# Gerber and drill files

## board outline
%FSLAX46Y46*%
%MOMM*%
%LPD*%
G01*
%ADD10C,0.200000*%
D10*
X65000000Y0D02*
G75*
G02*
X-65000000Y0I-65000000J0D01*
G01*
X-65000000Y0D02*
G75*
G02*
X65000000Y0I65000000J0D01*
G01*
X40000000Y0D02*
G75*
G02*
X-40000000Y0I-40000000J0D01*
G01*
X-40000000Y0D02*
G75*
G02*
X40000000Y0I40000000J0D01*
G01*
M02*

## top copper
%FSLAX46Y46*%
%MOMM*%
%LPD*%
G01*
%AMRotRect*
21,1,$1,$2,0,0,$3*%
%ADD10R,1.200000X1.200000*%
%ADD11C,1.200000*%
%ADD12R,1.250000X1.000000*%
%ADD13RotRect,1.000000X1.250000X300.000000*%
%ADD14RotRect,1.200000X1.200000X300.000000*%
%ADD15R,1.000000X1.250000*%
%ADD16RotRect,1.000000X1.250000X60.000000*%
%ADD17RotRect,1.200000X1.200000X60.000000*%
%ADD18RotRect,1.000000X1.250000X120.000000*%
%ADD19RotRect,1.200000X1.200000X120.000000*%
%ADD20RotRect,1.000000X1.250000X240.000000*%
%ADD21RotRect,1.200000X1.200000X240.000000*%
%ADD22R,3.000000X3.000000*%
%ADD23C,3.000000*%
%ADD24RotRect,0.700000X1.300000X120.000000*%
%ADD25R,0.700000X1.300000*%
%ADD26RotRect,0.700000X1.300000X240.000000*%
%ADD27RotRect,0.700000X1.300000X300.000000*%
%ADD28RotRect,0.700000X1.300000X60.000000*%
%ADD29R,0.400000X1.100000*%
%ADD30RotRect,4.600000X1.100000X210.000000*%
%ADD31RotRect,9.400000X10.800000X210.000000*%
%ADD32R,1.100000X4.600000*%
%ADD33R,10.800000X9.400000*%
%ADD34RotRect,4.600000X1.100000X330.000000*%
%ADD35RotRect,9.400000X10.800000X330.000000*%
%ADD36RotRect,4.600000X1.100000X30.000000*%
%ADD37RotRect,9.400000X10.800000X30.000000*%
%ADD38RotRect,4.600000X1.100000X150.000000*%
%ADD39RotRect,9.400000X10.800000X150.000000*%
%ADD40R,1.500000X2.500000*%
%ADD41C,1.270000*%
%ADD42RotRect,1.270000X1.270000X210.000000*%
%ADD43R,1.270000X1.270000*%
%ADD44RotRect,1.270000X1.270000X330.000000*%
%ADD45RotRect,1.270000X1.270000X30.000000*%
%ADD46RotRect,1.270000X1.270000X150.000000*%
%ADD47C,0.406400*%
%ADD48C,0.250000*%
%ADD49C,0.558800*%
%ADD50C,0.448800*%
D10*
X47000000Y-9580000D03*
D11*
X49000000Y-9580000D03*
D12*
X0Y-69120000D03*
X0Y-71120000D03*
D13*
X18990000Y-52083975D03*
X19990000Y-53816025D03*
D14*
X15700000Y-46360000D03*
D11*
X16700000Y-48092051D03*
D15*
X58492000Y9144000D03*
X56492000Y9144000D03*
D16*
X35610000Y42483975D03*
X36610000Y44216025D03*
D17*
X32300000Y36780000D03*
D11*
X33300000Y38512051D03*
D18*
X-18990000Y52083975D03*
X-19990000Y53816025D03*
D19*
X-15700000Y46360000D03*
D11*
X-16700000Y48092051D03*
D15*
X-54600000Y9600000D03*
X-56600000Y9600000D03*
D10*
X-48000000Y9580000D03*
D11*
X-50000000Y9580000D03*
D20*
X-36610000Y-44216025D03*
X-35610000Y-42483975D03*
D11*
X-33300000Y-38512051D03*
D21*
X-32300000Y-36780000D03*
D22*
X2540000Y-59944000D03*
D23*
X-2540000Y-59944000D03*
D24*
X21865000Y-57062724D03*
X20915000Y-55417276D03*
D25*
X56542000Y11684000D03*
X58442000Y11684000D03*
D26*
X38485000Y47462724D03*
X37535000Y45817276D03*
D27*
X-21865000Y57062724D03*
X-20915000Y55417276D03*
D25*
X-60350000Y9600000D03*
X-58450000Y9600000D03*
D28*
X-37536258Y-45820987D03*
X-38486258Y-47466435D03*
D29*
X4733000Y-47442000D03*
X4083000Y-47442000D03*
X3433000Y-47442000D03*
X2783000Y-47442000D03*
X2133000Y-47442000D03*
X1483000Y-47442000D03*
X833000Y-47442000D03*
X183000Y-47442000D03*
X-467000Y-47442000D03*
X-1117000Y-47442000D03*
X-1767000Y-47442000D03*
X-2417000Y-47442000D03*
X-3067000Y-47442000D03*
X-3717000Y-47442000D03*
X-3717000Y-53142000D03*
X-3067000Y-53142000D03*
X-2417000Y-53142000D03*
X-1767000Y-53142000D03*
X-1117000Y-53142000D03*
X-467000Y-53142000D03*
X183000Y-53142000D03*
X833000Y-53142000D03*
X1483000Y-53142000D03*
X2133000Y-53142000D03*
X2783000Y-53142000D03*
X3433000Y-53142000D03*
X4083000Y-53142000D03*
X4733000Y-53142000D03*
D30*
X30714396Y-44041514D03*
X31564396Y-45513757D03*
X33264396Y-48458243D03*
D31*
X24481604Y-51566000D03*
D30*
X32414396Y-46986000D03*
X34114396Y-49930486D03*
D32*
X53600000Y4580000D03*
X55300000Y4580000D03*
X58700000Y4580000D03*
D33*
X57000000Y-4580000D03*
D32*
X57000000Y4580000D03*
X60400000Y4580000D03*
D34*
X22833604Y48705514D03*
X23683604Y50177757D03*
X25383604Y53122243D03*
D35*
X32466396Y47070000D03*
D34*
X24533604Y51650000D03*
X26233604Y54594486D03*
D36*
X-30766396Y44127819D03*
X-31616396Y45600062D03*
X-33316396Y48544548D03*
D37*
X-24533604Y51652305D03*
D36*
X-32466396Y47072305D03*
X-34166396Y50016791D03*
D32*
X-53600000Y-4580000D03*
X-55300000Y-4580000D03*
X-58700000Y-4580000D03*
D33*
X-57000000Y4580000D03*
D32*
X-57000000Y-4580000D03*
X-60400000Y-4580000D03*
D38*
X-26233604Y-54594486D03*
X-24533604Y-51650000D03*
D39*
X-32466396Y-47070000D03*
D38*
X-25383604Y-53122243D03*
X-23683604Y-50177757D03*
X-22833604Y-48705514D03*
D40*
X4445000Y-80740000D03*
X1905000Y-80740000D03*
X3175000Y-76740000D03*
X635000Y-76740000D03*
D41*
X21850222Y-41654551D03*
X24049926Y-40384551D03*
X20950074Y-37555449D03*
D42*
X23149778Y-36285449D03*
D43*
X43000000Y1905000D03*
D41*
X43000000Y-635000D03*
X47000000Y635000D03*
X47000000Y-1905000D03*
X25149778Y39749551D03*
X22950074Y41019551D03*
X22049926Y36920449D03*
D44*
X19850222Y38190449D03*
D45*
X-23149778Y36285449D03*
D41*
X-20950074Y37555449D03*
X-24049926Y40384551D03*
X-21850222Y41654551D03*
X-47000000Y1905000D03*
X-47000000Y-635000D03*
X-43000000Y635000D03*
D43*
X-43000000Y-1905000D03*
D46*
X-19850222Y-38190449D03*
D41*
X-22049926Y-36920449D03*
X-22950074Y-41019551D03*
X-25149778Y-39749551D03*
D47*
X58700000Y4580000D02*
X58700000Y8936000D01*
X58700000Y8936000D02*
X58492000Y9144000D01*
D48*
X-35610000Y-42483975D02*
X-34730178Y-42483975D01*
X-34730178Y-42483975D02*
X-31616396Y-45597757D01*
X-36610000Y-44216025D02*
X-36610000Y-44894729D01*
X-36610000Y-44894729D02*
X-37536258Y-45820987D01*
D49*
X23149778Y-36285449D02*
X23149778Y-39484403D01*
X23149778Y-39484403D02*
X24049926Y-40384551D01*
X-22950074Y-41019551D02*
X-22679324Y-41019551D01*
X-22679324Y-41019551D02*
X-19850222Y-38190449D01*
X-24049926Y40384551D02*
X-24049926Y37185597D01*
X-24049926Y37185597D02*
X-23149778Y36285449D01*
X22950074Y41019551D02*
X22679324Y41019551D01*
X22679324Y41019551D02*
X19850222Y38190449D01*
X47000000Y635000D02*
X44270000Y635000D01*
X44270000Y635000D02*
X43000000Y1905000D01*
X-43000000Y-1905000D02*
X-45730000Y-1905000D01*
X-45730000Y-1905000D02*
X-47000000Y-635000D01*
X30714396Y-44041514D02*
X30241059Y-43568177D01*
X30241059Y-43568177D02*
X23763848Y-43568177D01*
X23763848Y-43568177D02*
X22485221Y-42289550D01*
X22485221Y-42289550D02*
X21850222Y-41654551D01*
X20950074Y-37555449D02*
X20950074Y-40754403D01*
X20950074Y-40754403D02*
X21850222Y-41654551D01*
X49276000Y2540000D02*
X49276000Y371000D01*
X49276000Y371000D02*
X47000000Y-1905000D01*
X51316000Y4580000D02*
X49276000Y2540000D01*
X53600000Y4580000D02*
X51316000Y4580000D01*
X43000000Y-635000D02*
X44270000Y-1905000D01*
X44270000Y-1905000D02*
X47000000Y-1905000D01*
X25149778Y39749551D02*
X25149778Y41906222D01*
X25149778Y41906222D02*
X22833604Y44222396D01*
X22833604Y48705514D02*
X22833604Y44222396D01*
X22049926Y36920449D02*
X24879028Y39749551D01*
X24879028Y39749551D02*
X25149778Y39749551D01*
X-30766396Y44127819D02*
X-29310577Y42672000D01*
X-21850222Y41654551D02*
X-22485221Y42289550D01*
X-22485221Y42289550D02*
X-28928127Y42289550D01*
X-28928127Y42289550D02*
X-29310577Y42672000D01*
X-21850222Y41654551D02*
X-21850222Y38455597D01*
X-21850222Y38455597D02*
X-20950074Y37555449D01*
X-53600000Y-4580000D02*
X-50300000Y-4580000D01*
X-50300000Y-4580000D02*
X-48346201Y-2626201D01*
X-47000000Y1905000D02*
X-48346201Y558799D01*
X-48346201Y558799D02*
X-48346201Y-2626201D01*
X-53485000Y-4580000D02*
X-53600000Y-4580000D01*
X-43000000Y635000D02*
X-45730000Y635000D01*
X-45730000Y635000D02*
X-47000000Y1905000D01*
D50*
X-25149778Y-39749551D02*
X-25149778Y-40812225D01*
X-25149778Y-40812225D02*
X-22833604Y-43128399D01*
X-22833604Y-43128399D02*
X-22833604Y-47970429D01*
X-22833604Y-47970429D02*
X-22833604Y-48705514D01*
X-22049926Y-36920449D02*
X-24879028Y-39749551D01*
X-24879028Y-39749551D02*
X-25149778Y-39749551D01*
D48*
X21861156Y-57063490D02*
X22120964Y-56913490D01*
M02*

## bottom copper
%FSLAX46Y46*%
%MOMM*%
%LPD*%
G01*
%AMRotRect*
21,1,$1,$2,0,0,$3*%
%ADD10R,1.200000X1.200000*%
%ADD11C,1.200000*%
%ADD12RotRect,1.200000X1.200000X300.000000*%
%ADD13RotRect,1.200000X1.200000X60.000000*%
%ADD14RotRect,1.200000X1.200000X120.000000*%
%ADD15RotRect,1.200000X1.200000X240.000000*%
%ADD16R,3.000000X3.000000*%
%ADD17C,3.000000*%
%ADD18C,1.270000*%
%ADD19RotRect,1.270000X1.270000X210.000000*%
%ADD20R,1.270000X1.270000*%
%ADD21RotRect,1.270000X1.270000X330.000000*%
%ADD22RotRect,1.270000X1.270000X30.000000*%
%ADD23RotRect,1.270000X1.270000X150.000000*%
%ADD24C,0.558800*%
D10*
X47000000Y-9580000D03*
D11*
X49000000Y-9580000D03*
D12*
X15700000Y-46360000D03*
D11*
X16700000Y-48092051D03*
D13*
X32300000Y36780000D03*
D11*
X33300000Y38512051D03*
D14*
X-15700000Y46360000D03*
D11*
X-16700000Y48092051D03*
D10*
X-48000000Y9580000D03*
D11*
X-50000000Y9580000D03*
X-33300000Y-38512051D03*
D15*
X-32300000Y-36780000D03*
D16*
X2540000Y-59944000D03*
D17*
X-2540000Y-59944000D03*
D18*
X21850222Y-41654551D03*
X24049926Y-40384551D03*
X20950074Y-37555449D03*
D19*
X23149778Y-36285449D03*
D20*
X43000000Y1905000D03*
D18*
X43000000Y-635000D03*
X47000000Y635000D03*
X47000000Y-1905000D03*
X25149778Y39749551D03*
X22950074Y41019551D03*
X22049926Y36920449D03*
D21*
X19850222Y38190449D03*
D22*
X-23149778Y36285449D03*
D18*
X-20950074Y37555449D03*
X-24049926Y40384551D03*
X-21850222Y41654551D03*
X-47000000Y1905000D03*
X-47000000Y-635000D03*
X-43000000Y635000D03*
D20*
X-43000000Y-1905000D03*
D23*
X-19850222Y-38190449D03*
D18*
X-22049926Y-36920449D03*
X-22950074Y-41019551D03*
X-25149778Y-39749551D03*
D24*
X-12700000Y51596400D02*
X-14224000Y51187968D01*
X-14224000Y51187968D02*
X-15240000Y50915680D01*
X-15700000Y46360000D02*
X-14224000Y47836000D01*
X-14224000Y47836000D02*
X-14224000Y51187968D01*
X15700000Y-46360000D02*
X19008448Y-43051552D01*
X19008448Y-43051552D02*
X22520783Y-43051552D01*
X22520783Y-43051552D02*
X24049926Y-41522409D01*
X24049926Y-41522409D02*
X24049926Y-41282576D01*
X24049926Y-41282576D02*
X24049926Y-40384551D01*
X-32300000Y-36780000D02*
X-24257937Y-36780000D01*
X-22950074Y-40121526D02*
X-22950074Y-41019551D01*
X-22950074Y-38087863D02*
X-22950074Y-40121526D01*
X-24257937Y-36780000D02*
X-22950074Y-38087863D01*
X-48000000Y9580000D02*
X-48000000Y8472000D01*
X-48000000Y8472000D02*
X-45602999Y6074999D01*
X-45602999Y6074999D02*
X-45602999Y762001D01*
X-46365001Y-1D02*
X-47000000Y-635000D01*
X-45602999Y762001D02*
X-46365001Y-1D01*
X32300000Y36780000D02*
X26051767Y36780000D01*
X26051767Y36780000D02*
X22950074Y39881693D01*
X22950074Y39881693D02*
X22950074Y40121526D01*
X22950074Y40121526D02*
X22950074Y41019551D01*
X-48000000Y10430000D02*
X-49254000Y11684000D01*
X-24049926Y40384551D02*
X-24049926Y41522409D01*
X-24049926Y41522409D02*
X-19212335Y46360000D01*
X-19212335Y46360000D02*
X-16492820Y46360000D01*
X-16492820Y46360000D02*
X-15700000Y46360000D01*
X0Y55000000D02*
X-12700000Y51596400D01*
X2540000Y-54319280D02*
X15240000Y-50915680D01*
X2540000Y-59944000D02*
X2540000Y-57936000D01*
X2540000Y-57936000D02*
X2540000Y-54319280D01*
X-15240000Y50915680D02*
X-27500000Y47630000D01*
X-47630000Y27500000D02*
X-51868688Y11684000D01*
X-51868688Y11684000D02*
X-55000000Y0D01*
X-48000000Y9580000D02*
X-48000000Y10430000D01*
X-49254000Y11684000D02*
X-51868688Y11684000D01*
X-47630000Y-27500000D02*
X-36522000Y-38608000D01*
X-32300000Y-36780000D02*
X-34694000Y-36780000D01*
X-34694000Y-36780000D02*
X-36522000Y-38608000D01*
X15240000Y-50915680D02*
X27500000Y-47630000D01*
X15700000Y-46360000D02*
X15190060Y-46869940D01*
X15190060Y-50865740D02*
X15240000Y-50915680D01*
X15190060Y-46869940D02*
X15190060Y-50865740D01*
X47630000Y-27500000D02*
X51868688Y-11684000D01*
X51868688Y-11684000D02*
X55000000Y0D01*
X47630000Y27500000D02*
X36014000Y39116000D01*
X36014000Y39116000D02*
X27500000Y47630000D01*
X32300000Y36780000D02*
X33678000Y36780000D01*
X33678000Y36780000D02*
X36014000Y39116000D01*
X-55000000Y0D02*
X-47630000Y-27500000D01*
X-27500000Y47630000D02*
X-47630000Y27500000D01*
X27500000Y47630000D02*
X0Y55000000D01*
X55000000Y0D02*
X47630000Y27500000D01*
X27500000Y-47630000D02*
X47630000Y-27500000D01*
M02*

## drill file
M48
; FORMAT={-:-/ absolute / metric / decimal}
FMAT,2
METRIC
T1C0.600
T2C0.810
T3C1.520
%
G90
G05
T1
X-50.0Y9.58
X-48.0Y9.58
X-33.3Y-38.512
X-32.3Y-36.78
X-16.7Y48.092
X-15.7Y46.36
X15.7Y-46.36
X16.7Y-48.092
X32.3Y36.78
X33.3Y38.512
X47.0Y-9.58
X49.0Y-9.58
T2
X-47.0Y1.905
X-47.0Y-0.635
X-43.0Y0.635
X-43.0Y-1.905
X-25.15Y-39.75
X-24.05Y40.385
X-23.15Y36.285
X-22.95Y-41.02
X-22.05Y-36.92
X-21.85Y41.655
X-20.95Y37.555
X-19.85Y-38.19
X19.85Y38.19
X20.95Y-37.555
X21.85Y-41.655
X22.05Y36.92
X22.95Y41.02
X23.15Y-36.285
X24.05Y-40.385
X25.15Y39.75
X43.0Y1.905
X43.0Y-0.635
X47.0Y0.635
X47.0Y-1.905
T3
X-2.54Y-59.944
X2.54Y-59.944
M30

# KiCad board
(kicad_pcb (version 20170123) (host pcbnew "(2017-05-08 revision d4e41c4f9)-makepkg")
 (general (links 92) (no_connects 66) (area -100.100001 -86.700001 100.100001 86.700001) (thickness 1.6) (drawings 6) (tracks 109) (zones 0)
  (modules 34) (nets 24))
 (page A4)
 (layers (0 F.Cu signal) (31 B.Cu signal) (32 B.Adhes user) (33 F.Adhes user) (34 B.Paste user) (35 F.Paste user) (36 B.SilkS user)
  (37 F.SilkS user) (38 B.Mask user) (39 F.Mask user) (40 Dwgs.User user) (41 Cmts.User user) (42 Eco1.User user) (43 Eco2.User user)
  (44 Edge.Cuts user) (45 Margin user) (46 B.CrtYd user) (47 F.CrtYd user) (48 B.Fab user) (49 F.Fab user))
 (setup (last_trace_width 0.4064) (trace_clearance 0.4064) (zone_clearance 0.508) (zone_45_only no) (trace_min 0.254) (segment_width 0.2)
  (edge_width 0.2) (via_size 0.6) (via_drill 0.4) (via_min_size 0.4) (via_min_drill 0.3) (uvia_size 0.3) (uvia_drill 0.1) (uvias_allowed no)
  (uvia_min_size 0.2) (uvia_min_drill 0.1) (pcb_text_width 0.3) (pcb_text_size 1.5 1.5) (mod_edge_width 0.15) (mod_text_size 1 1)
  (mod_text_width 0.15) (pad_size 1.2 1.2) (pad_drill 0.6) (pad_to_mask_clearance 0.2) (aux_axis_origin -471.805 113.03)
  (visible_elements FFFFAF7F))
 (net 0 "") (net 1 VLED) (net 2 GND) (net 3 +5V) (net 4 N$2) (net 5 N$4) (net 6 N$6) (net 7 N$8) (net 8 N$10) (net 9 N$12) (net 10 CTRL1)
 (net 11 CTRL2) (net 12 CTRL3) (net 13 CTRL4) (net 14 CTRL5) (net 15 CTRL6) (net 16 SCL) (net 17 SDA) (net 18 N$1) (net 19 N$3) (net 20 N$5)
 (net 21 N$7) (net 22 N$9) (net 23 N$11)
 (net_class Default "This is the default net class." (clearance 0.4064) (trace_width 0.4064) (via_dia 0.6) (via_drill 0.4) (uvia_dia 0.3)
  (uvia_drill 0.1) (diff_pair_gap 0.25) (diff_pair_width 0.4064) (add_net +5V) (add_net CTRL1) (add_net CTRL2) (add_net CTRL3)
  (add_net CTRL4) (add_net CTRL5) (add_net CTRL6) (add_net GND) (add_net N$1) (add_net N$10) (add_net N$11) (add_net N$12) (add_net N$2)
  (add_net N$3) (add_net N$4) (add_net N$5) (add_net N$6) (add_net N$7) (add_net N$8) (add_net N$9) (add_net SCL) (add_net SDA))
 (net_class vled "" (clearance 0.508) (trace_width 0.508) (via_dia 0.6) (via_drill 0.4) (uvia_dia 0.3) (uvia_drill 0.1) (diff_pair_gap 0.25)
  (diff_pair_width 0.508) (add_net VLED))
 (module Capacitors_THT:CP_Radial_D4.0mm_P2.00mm (layer F.Cu) (at 47 9.58)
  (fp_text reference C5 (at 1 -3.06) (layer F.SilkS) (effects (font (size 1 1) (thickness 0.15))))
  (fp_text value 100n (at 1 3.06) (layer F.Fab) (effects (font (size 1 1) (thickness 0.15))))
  (pad 1 thru_hole rect (at 0 0) (size 1.2 1.2) (drill 0.6) (layers *.Cu *.Mask) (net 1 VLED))
  (pad 2 thru_hole circle (at 2 0) (size 1.2 1.2) (drill 0.6) (layers *.Cu *.Mask) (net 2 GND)))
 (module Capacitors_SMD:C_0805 (layer F.Cu) (at 0 70.12 270)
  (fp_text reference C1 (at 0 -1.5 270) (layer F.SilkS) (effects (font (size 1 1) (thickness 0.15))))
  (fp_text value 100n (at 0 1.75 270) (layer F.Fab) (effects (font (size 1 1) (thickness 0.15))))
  (pad 1 smd rect (at -1 0 270) (size 1 1.25) (layers F.Cu F.Paste F.Mask) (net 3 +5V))
  (pad 2 smd rect (at 1 0 270) (size 1 1.25) (layers F.Cu F.Paste F.Mask) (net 2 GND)))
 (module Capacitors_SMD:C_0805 (layer F.Cu) (at 19.49 52.95 300)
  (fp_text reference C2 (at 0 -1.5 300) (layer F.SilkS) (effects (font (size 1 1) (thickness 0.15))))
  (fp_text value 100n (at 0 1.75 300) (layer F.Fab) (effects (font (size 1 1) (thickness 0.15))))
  (pad 1 smd rect (at -1 0 300) (size 1 1.25) (layers F.Cu F.Paste F.Mask) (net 3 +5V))
  (pad 2 smd rect (at 1 0 300) (size 1 1.25) (layers F.Cu F.Paste F.Mask) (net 2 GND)))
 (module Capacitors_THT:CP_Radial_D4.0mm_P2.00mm (layer F.Cu) (at 15.7 46.36 300)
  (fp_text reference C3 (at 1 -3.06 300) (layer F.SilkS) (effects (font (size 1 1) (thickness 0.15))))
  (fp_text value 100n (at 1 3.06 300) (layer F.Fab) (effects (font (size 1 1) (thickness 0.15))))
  (pad 1 thru_hole rect (at 0 0 300) (size 1.2 1.2) (drill 0.6) (layers *.Cu *.Mask) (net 1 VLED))
  (pad 2 thru_hole circle (at 2 0 300) (size 1.2 1.2) (drill 0.6) (layers *.Cu *.Mask) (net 2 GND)))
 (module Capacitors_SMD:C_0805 (layer F.Cu) (at 57.492 -9.144 180)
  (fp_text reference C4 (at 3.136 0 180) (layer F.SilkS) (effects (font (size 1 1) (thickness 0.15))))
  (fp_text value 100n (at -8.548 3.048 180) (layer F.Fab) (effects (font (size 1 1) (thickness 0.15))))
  (pad 1 smd rect (at -1 0 180) (size 1 1.25) (layers F.Cu F.Paste F.Mask) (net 3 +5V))
  (pad 2 smd rect (at 1 0 180) (size 1 1.25) (layers F.Cu F.Paste F.Mask) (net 2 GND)))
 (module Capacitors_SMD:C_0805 (layer F.Cu) (at 36.11 -43.35 60)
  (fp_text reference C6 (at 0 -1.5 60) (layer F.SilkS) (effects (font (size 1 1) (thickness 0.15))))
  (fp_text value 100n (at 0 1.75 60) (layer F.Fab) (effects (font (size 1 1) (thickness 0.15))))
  (pad 1 smd rect (at -1 0 60) (size 1 1.25) (layers F.Cu F.Paste F.Mask) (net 3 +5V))
  (pad 2 smd rect (at 1 0 60) (size 1 1.25) (layers F.Cu F.Paste F.Mask) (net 2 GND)))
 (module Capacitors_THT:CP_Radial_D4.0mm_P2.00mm (layer F.Cu) (at 32.3 -36.78 60)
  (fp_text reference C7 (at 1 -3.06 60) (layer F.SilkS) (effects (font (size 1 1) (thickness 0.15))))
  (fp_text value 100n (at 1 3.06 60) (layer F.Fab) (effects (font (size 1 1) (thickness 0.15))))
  (pad 1 thru_hole rect (at 0 0 60) (size 1.2 1.2) (drill 0.6) (layers *.Cu *.Mask) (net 1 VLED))
  (pad 2 thru_hole circle (at 2 0 60) (size 1.2 1.2) (drill 0.6) (layers *.Cu *.Mask) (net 2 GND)))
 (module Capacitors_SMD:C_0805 (layer F.Cu) (at -19.49 -52.95 120)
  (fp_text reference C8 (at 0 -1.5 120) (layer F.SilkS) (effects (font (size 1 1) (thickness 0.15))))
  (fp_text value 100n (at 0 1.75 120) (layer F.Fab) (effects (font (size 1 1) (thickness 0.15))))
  (pad 1 smd rect (at -1 0 120) (size 1 1.25) (layers F.Cu F.Paste F.Mask) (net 3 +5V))
  (pad 2 smd rect (at 1 0 120) (size 1 1.25) (layers F.Cu F.Paste F.Mask) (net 2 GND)))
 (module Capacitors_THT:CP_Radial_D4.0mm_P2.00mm (layer F.Cu) (at -15.7 -46.36 120)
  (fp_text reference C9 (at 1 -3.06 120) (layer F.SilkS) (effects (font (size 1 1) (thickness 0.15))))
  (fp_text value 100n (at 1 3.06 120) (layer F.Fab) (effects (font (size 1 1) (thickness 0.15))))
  (pad 1 thru_hole rect (at 0 0 120) (size 1.2 1.2) (drill 0.6) (layers *.Cu *.Mask) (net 1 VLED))
  (pad 2 thru_hole circle (at 2 0 120) (size 1.2 1.2) (drill 0.6) (layers *.Cu *.Mask) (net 2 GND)))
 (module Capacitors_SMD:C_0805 (layer F.Cu) (at -55.6 -9.6 180)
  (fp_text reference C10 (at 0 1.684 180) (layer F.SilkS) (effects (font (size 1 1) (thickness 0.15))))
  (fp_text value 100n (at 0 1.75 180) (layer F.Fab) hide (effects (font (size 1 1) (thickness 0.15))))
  (pad 1 smd rect (at -1 0 180) (size 1 1.25) (layers F.Cu F.Paste F.Mask) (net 3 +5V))
  (pad 2 smd rect (at 1 0 180) (size 1 1.25) (layers F.Cu F.Paste F.Mask) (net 2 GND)))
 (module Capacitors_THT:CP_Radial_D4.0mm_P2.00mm (layer F.Cu) (at -48 -9.58 180)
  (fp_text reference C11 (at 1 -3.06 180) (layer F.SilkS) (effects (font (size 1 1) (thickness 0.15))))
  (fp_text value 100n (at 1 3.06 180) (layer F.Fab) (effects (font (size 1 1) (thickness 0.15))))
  (pad 1 thru_hole rect (at 0 0 180) (size 1.2 1.2) (drill 0.6) (layers *.Cu *.Mask) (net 1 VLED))
  (pad 2 thru_hole circle (at 2 0 180) (size 1.2 1.2) (drill 0.6) (layers *.Cu *.Mask) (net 2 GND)))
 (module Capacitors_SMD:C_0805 (layer F.Cu) (at -36.11 43.35 240)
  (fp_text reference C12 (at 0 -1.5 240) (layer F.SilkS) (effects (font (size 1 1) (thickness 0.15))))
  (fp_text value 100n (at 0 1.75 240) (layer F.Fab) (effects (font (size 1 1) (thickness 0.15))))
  (pad 2 smd rect (at 1 0 240) (size 1 1.25) (layers F.Cu F.Paste F.Mask) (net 2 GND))
  (pad 1 smd rect (at -1 0 240) (size 1 1.25) (layers F.Cu F.Paste F.Mask) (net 3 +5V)))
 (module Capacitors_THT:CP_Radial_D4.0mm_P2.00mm (layer F.Cu) (at -32.3 36.78 240)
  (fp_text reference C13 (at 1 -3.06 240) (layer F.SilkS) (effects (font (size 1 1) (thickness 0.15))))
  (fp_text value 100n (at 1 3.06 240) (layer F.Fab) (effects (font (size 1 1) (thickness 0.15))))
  (pad 2 thru_hole circle (at 2 0 240) (size 1.2 1.2) (drill 0.6) (layers *.Cu *.Mask) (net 2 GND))
  (pad 1 thru_hole rect (at 0 0 240) (size 1.2 1.2) (drill 0.6) (layers *.Cu *.Mask) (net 1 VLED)))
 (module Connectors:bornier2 (layer F.Cu) (at 2.54 59.944 180)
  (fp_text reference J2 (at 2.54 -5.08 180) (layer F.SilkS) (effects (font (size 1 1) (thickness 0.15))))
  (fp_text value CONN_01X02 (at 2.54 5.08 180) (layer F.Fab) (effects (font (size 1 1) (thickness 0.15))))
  (pad 1 thru_hole rect (at 0 0 180) (size 3 3) (drill 1.52) (layers *.Cu *.Mask) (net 1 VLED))
  (pad 2 thru_hole circle (at 5.08 0 180) (size 3 3) (drill 1.52) (layers *.Cu *.Mask) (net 2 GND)))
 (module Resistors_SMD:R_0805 (layer F.Cu) (at 21.39 56.24 120)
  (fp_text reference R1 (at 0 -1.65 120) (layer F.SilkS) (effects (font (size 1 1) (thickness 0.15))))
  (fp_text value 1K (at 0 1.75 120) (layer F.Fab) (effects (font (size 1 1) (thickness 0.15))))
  (pad 1 smd rect (at -0.95 0 120) (size 0.7 1.3) (layers F.Cu F.Paste F.Mask) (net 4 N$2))
  (pad 2 smd rect (at 0.95 0 120) (size 0.7 1.3) (layers F.Cu F.Paste F.Mask) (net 2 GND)))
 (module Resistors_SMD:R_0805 (layer F.Cu) (at 57.492 -11.684)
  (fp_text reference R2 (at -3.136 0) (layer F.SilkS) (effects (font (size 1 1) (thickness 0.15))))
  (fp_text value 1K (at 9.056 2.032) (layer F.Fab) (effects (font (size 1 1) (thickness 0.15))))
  (pad 1 smd rect (at -0.95 0) (size 0.7 1.3) (layers F.Cu F.Paste F.Mask) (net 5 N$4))
  (pad 2 smd rect (at 0.95 0) (size 0.7 1.3) (layers F.Cu F.Paste F.Mask) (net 2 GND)))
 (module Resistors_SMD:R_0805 (layer F.Cu) (at 38.01 -46.64 240)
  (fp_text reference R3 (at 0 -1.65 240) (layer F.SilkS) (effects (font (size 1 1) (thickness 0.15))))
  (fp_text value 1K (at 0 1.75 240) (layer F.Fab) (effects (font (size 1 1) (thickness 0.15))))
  (pad 1 smd rect (at -0.95 0 240) (size 0.7 1.3) (layers F.Cu F.Paste F.Mask) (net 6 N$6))
  (pad 2 smd rect (at 0.95 0 240) (size 0.7 1.3) (layers F.Cu F.Paste F.Mask) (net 2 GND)))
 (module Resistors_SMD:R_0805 (layer F.Cu) (at -21.39 -56.24 300)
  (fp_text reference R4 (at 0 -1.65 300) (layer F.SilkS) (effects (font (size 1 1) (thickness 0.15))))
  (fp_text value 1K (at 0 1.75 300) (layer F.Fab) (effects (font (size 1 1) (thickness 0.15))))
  (pad 1 smd rect (at -0.95 0 300) (size 0.7 1.3) (layers F.Cu F.Paste F.Mask) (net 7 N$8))
  (pad 2 smd rect (at 0.95 0 300) (size 0.7 1.3) (layers F.Cu F.Paste F.Mask) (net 2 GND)))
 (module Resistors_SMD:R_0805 (layer F.Cu) (at -59.4 -9.6)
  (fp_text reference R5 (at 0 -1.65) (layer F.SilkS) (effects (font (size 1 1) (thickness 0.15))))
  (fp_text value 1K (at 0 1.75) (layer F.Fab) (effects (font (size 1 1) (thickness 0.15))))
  (pad 1 smd rect (at -0.95 0) (size 0.7 1.3) (layers F.Cu F.Paste F.Mask) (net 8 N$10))
  (pad 2 smd rect (at 0.95 0) (size 0.7 1.3) (layers F.Cu F.Paste F.Mask) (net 2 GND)))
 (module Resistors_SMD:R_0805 (layer F.Cu) (at -38.011258 46.643711 60)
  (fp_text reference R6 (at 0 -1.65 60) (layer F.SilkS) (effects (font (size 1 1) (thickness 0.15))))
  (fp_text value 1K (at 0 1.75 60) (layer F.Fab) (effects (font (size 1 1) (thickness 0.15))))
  (pad 2 smd rect (at 0.95 0 60) (size 0.7 1.3) (layers F.Cu F.Paste F.Mask) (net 2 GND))
  (pad 1 smd rect (at -0.95 0 60) (size 0.7 1.3) (layers F.Cu F.Paste F.Mask) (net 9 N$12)))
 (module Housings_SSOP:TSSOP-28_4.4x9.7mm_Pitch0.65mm (layer F.Cu) (at 0.508 50.292 270)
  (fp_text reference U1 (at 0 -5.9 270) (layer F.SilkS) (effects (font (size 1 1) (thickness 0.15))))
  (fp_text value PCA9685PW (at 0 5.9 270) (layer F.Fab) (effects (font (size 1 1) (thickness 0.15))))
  (pad 1 smd rect (at -2.85 -4.225 270) (size 1.1 0.4) (layers F.Cu F.Paste F.Mask))
  (pad 2 smd rect (at -2.85 -3.575 270) (size 1.1 0.4) (layers F.Cu F.Paste F.Mask))
  (pad 3 smd rect (at -2.85 -2.925 270) (size 1.1 0.4) (layers F.Cu F.Paste F.Mask))
  (pad 4 smd rect (at -2.85 -2.275 270) (size 1.1 0.4) (layers F.Cu F.Paste F.Mask))
  (pad 5 smd rect (at -2.85 -1.625 270) (size 1.1 0.4) (layers F.Cu F.Paste F.Mask))
  (pad 6 smd rect (at -2.85 -0.975 270) (size 1.1 0.4) (layers F.Cu F.Paste F.Mask) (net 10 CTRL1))
  (pad 7 smd rect (at -2.85 -0.325 270) (size 1.1 0.4) (layers F.Cu F.Paste F.Mask) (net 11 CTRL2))
  (pad 8 smd rect (at -2.85 0.325 270) (size 1.1 0.4) (layers F.Cu F.Paste F.Mask) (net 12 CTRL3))
  (pad 9 smd rect (at -2.85 0.975 270) (size 1.1 0.4) (layers F.Cu F.Paste F.Mask) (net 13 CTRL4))
  (pad 10 smd rect (at -2.85 1.625 270) (size 1.1 0.4) (layers F.Cu F.Paste F.Mask) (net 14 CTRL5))
  (pad 11 smd rect (at -2.85 2.275 270) (size 1.1 0.4) (layers F.Cu F.Paste F.Mask) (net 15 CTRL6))
  (pad 12 smd rect (at -2.85 2.925 270) (size 1.1 0.4) (layers F.Cu F.Paste F.Mask))
  (pad 13 smd rect (at -2.85 3.575 270) (size 1.1 0.4) (layers F.Cu F.Paste F.Mask))
  (pad 14 smd rect (at -2.85 4.225 270) (size 1.1 0.4) (layers F.Cu F.Paste F.Mask) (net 2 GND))
  (pad 15 smd rect (at 2.85 4.225 270) (size 1.1 0.4) (layers F.Cu F.Paste F.Mask))
  (pad 16 smd rect (at 2.85 3.575 270) (size 1.1 0.4) (layers F.Cu F.Paste F.Mask))
  (pad 17 smd rect (at 2.85 2.925 270) (size 1.1 0.4) (layers F.Cu F.Paste F.Mask))
  (pad 18 smd rect (at 2.85 2.275 270) (size 1.1 0.4) (layers F.Cu F.Paste F.Mask))
  (pad 19 smd rect (at 2.85 1.625 270) (size 1.1 0.4) (layers F.Cu F.Paste F.Mask))
  (pad 20 smd rect (at 2.85 0.975 270) (size 1.1 0.4) (layers F.Cu F.Paste F.Mask))
  (pad 21 smd rect (at 2.85 0.325 270) (size 1.1 0.4) (layers F.Cu F.Paste F.Mask))
  (pad 22 smd rect (at 2.85 -0.325 270) (size 1.1 0.4) (layers F.Cu F.Paste F.Mask))
  (pad 23 smd rect (at 2.85 -0.975 270) (size 1.1 0.4) (layers F.Cu F.Paste F.Mask) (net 2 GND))
  (pad 24 smd rect (at 2.85 -1.625 270) (size 1.1 0.4) (layers F.Cu F.Paste F.Mask))
  (pad 25 smd rect (at 2.85 -2.275 270) (size 1.1 0.4) (layers F.Cu F.Paste F.Mask))
  (pad 26 smd rect (at 2.85 -2.925 270) (size 1.1 0.4) (layers F.Cu F.Paste F.Mask) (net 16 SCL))
  (pad 27 smd rect (at 2.85 -3.575 270) (size 1.1 0.4) (layers F.Cu F.Paste F.Mask) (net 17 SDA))
  (pad 28 smd rect (at 2.85 -4.225 270) (size 1.1 0.4) (layers F.Cu F.Paste F.Mask) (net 3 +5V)))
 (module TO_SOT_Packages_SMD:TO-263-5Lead (layer F.Cu) (at 28.448 49.276 210)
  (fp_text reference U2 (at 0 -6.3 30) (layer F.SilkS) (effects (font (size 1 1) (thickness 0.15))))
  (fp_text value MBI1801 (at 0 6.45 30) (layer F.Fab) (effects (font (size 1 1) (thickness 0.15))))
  (pad 5 smd rect (at -4.58 3.4 210) (size 4.6 1.1) (layers F.Cu F.Paste F.Mask) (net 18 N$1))
  (pad 4 smd rect (at -4.58 1.7 210) (size 4.6 1.1) (layers F.Cu F.Paste F.Mask) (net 4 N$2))
  (pad 2 smd rect (at -4.58 -1.7 210) (size 4.6 1.1) (layers F.Cu F.Paste F.Mask) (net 3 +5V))
  (pad 3 smd rect (at 4.58 0 210) (size 9.4 10.8) (layers F.Cu F.Paste F.Mask) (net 2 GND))
  (pad 3 smd rect (at -4.58 0 210) (size 4.6 1.1) (layers F.Cu F.Paste F.Mask) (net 2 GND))
  (pad 1 smd rect (at -4.58 -3.4 210) (size 4.6 1.1) (layers F.Cu F.Paste F.Mask) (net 10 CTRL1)))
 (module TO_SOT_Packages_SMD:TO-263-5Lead (layer F.Cu) (at 57 0 270)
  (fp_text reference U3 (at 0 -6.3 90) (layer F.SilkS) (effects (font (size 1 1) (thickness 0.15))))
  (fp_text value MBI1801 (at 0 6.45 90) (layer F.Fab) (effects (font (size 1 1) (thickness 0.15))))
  (pad 5 smd rect (at -4.58 3.4 270) (size 4.6 1.1) (layers F.Cu F.Paste F.Mask) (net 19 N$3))
  (pad 4 smd rect (at -4.58 1.7 270) (size 4.6 1.1) (layers F.Cu F.Paste F.Mask) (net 5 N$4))
  (pad 2 smd rect (at -4.58 -1.7 270) (size 4.6 1.1) (layers F.Cu F.Paste F.Mask) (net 3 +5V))
  (pad 3 smd rect (at 4.58 0 270) (size 9.4 10.8) (layers F.Cu F.Paste F.Mask) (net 2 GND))
  (pad 3 smd rect (at -4.58 0 270) (size 4.6 1.1) (layers F.Cu F.Paste F.Mask) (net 2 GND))
  (pad 1 smd rect (at -4.58 -3.4 270) (size 4.6 1.1) (layers F.Cu F.Paste F.Mask) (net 11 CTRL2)))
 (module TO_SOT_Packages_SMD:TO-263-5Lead (layer F.Cu) (at 28.5 -49.36 330)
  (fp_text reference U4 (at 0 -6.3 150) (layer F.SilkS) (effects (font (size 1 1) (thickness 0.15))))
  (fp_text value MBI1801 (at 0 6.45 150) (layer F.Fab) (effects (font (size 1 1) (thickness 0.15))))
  (pad 5 smd rect (at -4.58 3.4 330) (size 4.6 1.1) (layers F.Cu F.Paste F.Mask) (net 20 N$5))
  (pad 4 smd rect (at -4.58 1.7 330) (size 4.6 1.1) (layers F.Cu F.Paste F.Mask) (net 6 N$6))
  (pad 2 smd rect (at -4.58 -1.7 330) (size 4.6 1.1) (layers F.Cu F.Paste F.Mask) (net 3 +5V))
  (pad 3 smd rect (at 4.58 0 330) (size 9.4 10.8) (layers F.Cu F.Paste F.Mask) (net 2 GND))
  (pad 3 smd rect (at -4.58 0 330) (size 4.6 1.1) (layers F.Cu F.Paste F.Mask) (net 2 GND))
  (pad 1 smd rect (at -4.58 -3.4 330) (size 4.6 1.1) (layers F.Cu F.Paste F.Mask) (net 12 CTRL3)))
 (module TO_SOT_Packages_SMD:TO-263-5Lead (layer F.Cu) (at -28.5 -49.362305 30)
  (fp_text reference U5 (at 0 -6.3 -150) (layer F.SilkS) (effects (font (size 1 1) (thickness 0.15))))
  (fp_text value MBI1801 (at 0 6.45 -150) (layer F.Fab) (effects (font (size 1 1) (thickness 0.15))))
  (pad 5 smd rect (at -4.58 3.4 30) (size 4.6 1.1) (layers F.Cu F.Paste F.Mask) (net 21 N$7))
  (pad 4 smd rect (at -4.58 1.7 30) (size 4.6 1.1) (layers F.Cu F.Paste F.Mask) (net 7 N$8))
  (pad 2 smd rect (at -4.58 -1.7 30) (size 4.6 1.1) (layers F.Cu F.Paste F.Mask) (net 3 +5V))
  (pad 3 smd rect (at 4.58 0 30) (size 9.4 10.8) (layers F.Cu F.Paste F.Mask) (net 2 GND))
  (pad 3 smd rect (at -4.58 0 30) (size 4.6 1.1) (layers F.Cu F.Paste F.Mask) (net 2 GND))
  (pad 1 smd rect (at -4.58 -3.4 30) (size 4.6 1.1) (layers F.Cu F.Paste F.Mask) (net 13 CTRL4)))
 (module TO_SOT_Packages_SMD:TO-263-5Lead (layer F.Cu) (at -57 0 90)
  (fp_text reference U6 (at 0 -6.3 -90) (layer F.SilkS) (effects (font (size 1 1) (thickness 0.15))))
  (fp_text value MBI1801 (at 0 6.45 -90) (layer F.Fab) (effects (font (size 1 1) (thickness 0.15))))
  (pad 5 smd rect (at -4.58 3.4 90) (size 4.6 1.1) (layers F.Cu F.Paste F.Mask) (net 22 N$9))
  (pad 4 smd rect (at -4.58 1.7 90) (size 4.6 1.1) (layers F.Cu F.Paste F.Mask) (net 8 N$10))
  (pad 2 smd rect (at -4.58 -1.7 90) (size 4.6 1.1) (layers F.Cu F.Paste F.Mask) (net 3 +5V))
  (pad 3 smd rect (at 4.58 0 90) (size 9.4 10.8) (layers F.Cu F.Paste F.Mask) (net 2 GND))
  (pad 3 smd rect (at -4.58 0 90) (size 4.6 1.1) (layers F.Cu F.Paste F.Mask) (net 2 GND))
  (pad 1 smd rect (at -4.58 -3.4 90) (size 4.6 1.1) (layers F.Cu F.Paste F.Mask) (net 14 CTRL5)))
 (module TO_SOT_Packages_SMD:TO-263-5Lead (layer F.Cu) (at -28.5 49.36 150)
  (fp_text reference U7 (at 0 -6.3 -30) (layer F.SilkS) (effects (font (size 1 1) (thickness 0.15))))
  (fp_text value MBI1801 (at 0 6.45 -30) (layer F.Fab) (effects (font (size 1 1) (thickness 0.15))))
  (pad 1 smd rect (at -4.58 -3.4 150) (size 4.6 1.1) (layers F.Cu F.Paste F.Mask) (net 15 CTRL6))
  (pad 3 smd rect (at -4.58 0 150) (size 4.6 1.1) (layers F.Cu F.Paste F.Mask) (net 2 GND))
  (pad 3 smd rect (at 4.58 0 150) (size 9.4 10.8) (layers F.Cu F.Paste F.Mask) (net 2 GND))
  (pad 2 smd rect (at -4.58 -1.7 150) (size 4.6 1.1) (layers F.Cu F.Paste F.Mask) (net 3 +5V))
  (pad 4 smd rect (at -4.58 1.7 150) (size 4.6 1.1) (layers F.Cu F.Paste F.Mask) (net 9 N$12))
  (pad 5 smd rect (at -4.58 3.4 150) (size 4.6 1.1) (layers F.Cu F.Paste F.Mask) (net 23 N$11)))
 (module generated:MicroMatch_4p (layer F.Cu) (at 2.54 78.74 180)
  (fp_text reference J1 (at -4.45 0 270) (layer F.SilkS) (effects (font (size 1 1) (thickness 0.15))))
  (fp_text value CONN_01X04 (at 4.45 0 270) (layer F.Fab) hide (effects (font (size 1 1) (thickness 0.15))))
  (pad 1 smd rect (at -1.905 -2 180) (size 1.5 2.5) (layers F.Cu F.Paste F.Mask) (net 17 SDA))
  (pad 3 smd rect (at 0.635 -2 180) (size 1.5 2.5) (layers F.Cu F.Paste F.Mask) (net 2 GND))
  (pad 2 smd rect (at -0.635 2 180) (size 1.5 2.5) (layers F.Cu F.Paste F.Mask) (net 16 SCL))
  (pad 4 smd rect (at 1.905 2 180) (size 1.5 2.5) (layers F.Cu F.Paste F.Mask) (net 3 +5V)))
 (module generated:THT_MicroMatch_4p (layer B.Cu) (at 22.5 38.97 210)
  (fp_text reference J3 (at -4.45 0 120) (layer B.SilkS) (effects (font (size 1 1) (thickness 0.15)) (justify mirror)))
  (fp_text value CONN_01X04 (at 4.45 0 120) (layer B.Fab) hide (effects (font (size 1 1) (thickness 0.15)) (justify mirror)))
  (pad 4 thru_hole circle (at 1.905 -2 210) (size 1.27 1.27) (drill 0.81) (layers *.Cu *.Mask) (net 18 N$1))
  (pad 2 thru_hole circle (at -0.635 -2 210) (size 1.27 1.27) (drill 0.81) (layers *.Cu *.Mask) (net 1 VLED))
  (pad 3 thru_hole circle (at 0.635 2 210) (size 1.27 1.27) (drill 0.81) (layers *.Cu *.Mask) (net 18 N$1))
  (pad 1 thru_hole rect (at -1.905 2 210) (size 1.27 1.27) (drill 0.81) (layers *.Cu *.Mask) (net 1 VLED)))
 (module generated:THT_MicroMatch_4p (layer B.Cu) (at 45 0 270)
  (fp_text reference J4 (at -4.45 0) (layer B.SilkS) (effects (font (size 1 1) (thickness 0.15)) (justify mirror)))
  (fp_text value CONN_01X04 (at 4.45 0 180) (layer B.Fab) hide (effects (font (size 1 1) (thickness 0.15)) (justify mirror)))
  (pad 1 thru_hole rect (at -1.905 2 270) (size 1.27 1.27) (drill 0.81) (layers *.Cu *.Mask) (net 1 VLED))
  (pad 3 thru_hole circle (at 0.635 2 270) (size 1.27 1.27) (drill 0.81) (layers *.Cu *.Mask) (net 19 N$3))
  (pad 2 thru_hole circle (at -0.635 -2 270) (size 1.27 1.27) (drill 0.81) (layers *.Cu *.Mask) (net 1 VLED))
  (pad 4 thru_hole circle (at 1.905 -2 270) (size 1.27 1.27) (drill 0.81) (layers *.Cu *.Mask) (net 19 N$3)))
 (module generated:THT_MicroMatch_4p (layer B.Cu) (at 22.5 -38.97 330)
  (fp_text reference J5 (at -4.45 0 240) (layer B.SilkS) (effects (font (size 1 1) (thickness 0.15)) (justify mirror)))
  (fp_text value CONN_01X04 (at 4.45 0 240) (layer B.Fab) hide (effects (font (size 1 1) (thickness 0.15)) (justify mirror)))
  (pad 4 thru_hole circle (at 1.905 -2 330) (size 1.27 1.27) (drill 0.81) (layers *.Cu *.Mask) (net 20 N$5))
  (pad 2 thru_hole circle (at -0.635 -2 330) (size 1.27 1.27) (drill 0.81) (layers *.Cu *.Mask) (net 1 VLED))
  (pad 3 thru_hole circle (at 0.635 2 330) (size 1.27 1.27) (drill 0.81) (layers *.Cu *.Mask) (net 20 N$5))
  (pad 1 thru_hole rect (at -1.905 2 330) (size 1.27 1.27) (drill 0.81) (layers *.Cu *.Mask) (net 1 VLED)))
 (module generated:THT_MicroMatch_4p (layer B.Cu) (at -22.5 -38.97 30)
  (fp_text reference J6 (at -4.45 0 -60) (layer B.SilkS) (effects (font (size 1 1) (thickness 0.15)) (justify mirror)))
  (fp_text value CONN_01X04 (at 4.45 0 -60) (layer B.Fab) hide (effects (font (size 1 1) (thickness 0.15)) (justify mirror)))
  (pad 1 thru_hole rect (at -1.905 2 30) (size 1.27 1.27) (drill 0.81) (layers *.Cu *.Mask) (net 1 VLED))
  (pad 3 thru_hole circle (at 0.635 2 30) (size 1.27 1.27) (drill 0.81) (layers *.Cu *.Mask) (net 21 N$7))
  (pad 2 thru_hole circle (at -0.635 -2 30) (size 1.27 1.27) (drill 0.81) (layers *.Cu *.Mask) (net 1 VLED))
  (pad 4 thru_hole circle (at 1.905 -2 30) (size 1.27 1.27) (drill 0.81) (layers *.Cu *.Mask) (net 21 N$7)))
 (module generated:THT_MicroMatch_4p (layer B.Cu) (at -45 0 90)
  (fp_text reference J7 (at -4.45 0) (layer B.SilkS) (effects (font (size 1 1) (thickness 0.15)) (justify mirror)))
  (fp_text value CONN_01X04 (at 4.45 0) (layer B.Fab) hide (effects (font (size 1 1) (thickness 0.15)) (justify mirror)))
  (pad 4 thru_hole circle (at 1.905 -2 90) (size 1.27 1.27) (drill 0.81) (layers *.Cu *.Mask) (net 22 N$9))
  (pad 2 thru_hole circle (at -0.635 -2 90) (size 1.27 1.27) (drill 0.81) (layers *.Cu *.Mask) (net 1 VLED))
  (pad 3 thru_hole circle (at 0.635 2 90) (size 1.27 1.27) (drill 0.81) (layers *.Cu *.Mask) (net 22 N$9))
  (pad 1 thru_hole rect (at -1.905 2 90) (size 1.27 1.27) (drill 0.81) (layers *.Cu *.Mask) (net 1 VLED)))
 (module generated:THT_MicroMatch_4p (layer B.Cu) (at -22.5 38.97 150)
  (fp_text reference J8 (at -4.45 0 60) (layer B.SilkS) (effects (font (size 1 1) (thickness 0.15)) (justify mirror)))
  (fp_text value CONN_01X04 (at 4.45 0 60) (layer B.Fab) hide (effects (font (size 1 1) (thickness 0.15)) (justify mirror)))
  (pad 1 thru_hole rect (at -1.905 2 150) (size 1.27 1.27) (drill 0.81) (layers *.Cu *.Mask) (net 1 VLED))
  (pad 3 thru_hole circle (at 0.635 2 150) (size 1.27 1.27) (drill 0.81) (layers *.Cu *.Mask) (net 23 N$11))
  (pad 2 thru_hole circle (at -0.635 -2 150) (size 1.27 1.27) (drill 0.81) (layers *.Cu *.Mask) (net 1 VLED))
  (pad 4 thru_hole circle (at 1.905 -2 150) (size 1.27 1.27) (drill 0.81) (layers *.Cu *.Mask) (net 23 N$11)))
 (gr_circle (center 0 0) (end 65 0) (layer Edge.Cuts) (width 0.2))
 (gr_circle (center 0 0) (end 40 0) (layer Edge.Cuts) (width 0.2))
 (segment (start 58.7 -4.58) (end 58.7 -8.936) (width 0.4064) (layer F.Cu) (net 3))
 (segment (start 58.7 -8.936) (end 58.492 -9.144) (width 0.4064) (layer F.Cu) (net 3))
 (segment (start -35.61 42.483975) (end -34.730178 42.483975) (width 0.25) (layer F.Cu) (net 3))
 (segment (start -34.730178 42.483975) (end -31.616396 45.597757) (width 0.25) (layer F.Cu) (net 2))
 (segment (start -36.61 44.216025) (end -36.61 44.894729) (width 0.25) (layer F.Cu) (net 2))
 (segment (start -36.61 44.894729) (end -37.536258 45.820987) (width 0.25) (layer F.Cu) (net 2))
 (segment (start 23.149778 36.285449) (end 23.149778 39.484403) (width 0.5588) (layer F.Cu) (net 1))
 (segment (start 23.149778 39.484403) (end 24.049926 40.384551) (width 0.5588) (layer F.Cu) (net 1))
 (segment (start -22.950074 41.019551) (end -22.679324 41.019551) (width 0.5588) (layer F.Cu) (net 1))
 (segment (start -22.679324 41.019551) (end -19.850222 38.190449) (width 0.5588) (layer F.Cu) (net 1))
 (segment (start -24.049926 -40.384551) (end -24.049926 -37.185597) (width 0.5588) (layer F.Cu) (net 1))
 (segment (start -24.049926 -37.185597) (end -23.149778 -36.285449) (width 0.5588) (layer F.Cu) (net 1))
 (segment (start 22.950074 -41.019551) (end 22.679324 -41.019551) (width 0.5588) (layer F.Cu) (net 1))
 (segment (start 22.679324 -41.019551) (end 19.850222 -38.190449) (width 0.5588) (layer F.Cu) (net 1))
 (segment (start 47 -0.635) (end 44.27 -0.635) (width 0.5588) (layer F.Cu) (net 1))
 (segment (start 44.27 -0.635) (end 43 -1.905) (width 0.5588) (layer F.Cu) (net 1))
 (segment (start -43 1.905) (end -45.73 1.905) (width 0.5588) (layer F.Cu) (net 1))
 (segment (start -45.73 1.905) (end -47 0.635) (width 0.5588) (layer F.Cu) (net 1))
 (segment (start -12.7 -51.5964) (end -14.224 -51.187968) (width 0.5588) (layer B.Cu) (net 1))
 (segment (start -14.224 -51.187968) (end -15.24 -50.91568) (width 0.5588) (layer B.Cu) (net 1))
 (segment (start -15.7 -46.36) (end -14.224 -47.836) (width 0.5588) (layer B.Cu) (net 1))
 (segment (start -14.224 -47.836) (end -14.224 -51.187968) (width 0.5588) (layer B.Cu) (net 1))
 (segment (start 15.7 46.36) (end 19.008448 43.051552) (width 0.5588) (layer B.Cu) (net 1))
 (segment (start 19.008448 43.051552) (end 22.520783 43.051552) (width 0.5588) (layer B.Cu) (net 1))
 (segment (start 22.520783 43.051552) (end 24.049926 41.522409) (width 0.5588) (layer B.Cu) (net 1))
 (segment (start 24.049926 41.522409) (end 24.049926 41.282576) (width 0.5588) (layer B.Cu) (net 1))
 (segment (start 24.049926 41.282576) (end 24.049926 40.384551) (width 0.5588) (layer B.Cu) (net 1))
 (segment (start -32.3 36.78) (end -24.257937 36.78) (width 0.5588) (layer B.Cu) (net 1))
 (segment (start -22.950074 40.121526) (end -22.950074 41.019551) (width 0.5588) (layer B.Cu) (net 1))
 (segment (start -22.950074 38.087863) (end -22.950074 40.121526) (width 0.5588) (layer B.Cu) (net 1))
 (segment (start -24.257937 36.78) (end -22.950074 38.087863) (width 0.5588) (layer B.Cu) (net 1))
 (segment (start -48 -9.58) (end -48 -8.472) (width 0.5588) (layer B.Cu) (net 1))
 (segment (start -48 -8.472) (end -45.602999 -6.074999) (width 0.5588) (layer B.Cu) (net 1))
 (segment (start -45.602999 -6.074999) (end -45.602999 -0.762001) (width 0.5588) (layer B.Cu) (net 1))
 (segment (start -46.365001 0.000001) (end -47 0.635) (width 0.5588) (layer B.Cu) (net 1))
 (segment (start -45.602999 -0.762001) (end -46.365001 0.000001) (width 0.5588) (layer B.Cu) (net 1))
 (segment (start 32.3 -36.78) (end 26.051767 -36.78) (width 0.5588) (layer B.Cu) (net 1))
 (segment (start 26.051767 -36.78) (end 22.950074 -39.881693) (width 0.5588) (layer B.Cu) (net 1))
 (segment (start 22.950074 -39.881693) (end 22.950074 -40.121526) (width 0.5588) (layer B.Cu) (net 1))
 (segment (start 22.950074 -40.121526) (end 22.950074 -41.019551) (width 0.5588) (layer B.Cu) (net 1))
 (segment (start -48 -10.43) (end -49.254 -11.684) (width 0.5588) (layer B.Cu) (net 1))
 (segment (start -24.049926 -40.384551) (end -24.049926 -41.522409) (width 0.5588) (layer B.Cu) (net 1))
 (segment (start -24.049926 -41.522409) (end -19.212335 -46.36) (width 0.5588) (layer B.Cu) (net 1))
 (segment (start -19.212335 -46.36) (end -16.49282 -46.36) (width 0.5588) (layer B.Cu) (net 1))
 (segment (start -16.49282 -46.36) (end -15.7 -46.36) (width 0.5588) (layer B.Cu) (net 1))
 (segment (start 0 -55) (end -12.7 -51.5964) (width 0.5588) (layer B.Cu) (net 1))
 (segment (start 2.54 54.31928) (end 15.24 50.91568) (width 0.5588) (layer B.Cu) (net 1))
 (segment (start 2.54 59.944) (end 2.54 57.936) (width 0.5588) (layer B.Cu) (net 1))
 (segment (start 2.54 57.936) (end 2.54 54.31928) (width 0.5588) (layer B.Cu) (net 1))
 (segment (start -15.24 -50.91568) (end -27.5 -47.63) (width 0.5588) (layer B.Cu) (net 1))
 (segment (start -47.63 -27.5) (end -51.868688 -11.684) (width 0.5588) (layer B.Cu) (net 1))
 (segment (start -51.868688 -11.684) (end -55 0) (width 0.5588) (layer B.Cu) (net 1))
 (segment (start -48 -9.58) (end -48 -10.43) (width 0.5588) (layer B.Cu) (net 1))
 (segment (start -49.254 -11.684) (end -51.868688 -11.684) (width 0.5588) (layer B.Cu) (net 1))
 (segment (start -47.63 27.5) (end -36.522 38.608) (width 0.5588) (layer B.Cu) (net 1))
 (segment (start -32.3 36.78) (end -34.694 36.78) (width 0.5588) (layer B.Cu) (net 1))
 (segment (start -34.694 36.78) (end -36.522 38.608) (width 0.5588) (layer B.Cu) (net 1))
 (segment (start 15.24 50.91568) (end 27.5 47.63) (width 0.5588) (layer B.Cu) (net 1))
 (segment (start 15.7 46.36) (end 15.19006 46.86994) (width 0.5588) (layer B.Cu) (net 1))
 (segment (start 15.19006 50.86574) (end 15.24 50.91568) (width 0.5588) (layer B.Cu) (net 1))
 (segment (start 15.19006 46.86994) (end 15.19006 50.86574) (width 0.5588) (layer B.Cu) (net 1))
 (segment (start 47.63 27.5) (end 51.868688 11.684) (width 0.5588) (layer B.Cu) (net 1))
 (segment (start 51.868688 11.684) (end 55 0) (width 0.5588) (layer B.Cu) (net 1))
 (segment (start 47.63 -27.5) (end 36.014 -39.116) (width 0.5588) (layer B.Cu) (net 1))
 (segment (start 36.014 -39.116) (end 27.5 -47.63) (width 0.5588) (layer B.Cu) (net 1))
 (segment (start 32.3 -36.78) (end 33.678 -36.78) (width 0.5588) (layer B.Cu) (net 1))
 (segment (start 33.678 -36.78) (end 36.014 -39.116) (width 0.5588) (layer B.Cu) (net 1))
 (segment (start -55 0) (end -47.63 27.5) (width 0.5588) (layer B.Cu) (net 1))
 (segment (start -27.5 -47.63) (end -47.63 -27.5) (width 0.5588) (layer B.Cu) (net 1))
 (segment (start 27.5 -47.63) (end 0 -55) (width 0.5588) (layer B.Cu) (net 1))
 (segment (start 55 0) (end 47.63 -27.5) (width 0.5588) (layer B.Cu) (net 1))
 (segment (start 27.5 47.63) (end 47.63 27.5) (width 0.5588) (layer B.Cu) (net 1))
 (segment (start 30.714396 44.041514) (end 30.241059 43.568177) (width 0.5588) (layer F.Cu) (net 18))
 (segment (start 30.241059 43.568177) (end 23.763848 43.568177) (width 0.5588) (layer F.Cu) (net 18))
 (segment (start 23.763848 43.568177) (end 22.485221 42.28955) (width 0.5588) (layer F.Cu) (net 18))
 (segment (start 22.485221 42.28955) (end 21.850222 41.654551) (width 0.5588) (layer F.Cu) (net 18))
 (segment (start 20.950074 37.555449) (end 20.950074 40.754403) (width 0.5588) (layer F.Cu) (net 18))
 (segment (start 20.950074 40.754403) (end 21.850222 41.654551) (width 0.5588) (layer F.Cu) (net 18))
 (segment (start 49.276 -2.54) (end 49.276 -0.371) (width 0.5588) (layer F.Cu) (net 19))
 (segment (start 49.276 -0.371) (end 47 1.905) (width 0.5588) (layer F.Cu) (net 19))
 (segment (start 51.316 -4.58) (end 49.276 -2.54) (width 0.5588) (layer F.Cu) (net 19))
 (segment (start 53.6 -4.58) (end 51.316 -4.58) (width 0.5588) (layer F.Cu) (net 19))
 (segment (start 43 0.635) (end 44.27 1.905) (width 0.5588) (layer F.Cu) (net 19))
 (segment (start 44.27 1.905) (end 47 1.905) (width 0.5588) (layer F.Cu) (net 19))
 (segment (start 25.149778 -39.749551) (end 25.149778 -41.906222) (width 0.5588) (layer F.Cu) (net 20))
 (segment (start 25.149778 -41.906222) (end 22.833604 -44.222396) (width 0.5588) (layer F.Cu) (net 20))
 (segment (start 22.833604 -48.705514) (end 22.833604 -44.222396) (width 0.5588) (layer F.Cu) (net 20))
 (segment (start 22.049926 -36.920449) (end 24.879028 -39.749551) (width 0.5588) (layer F.Cu) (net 20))
 (segment (start 24.879028 -39.749551) (end 25.149778 -39.749551) (width 0.5588) (layer F.Cu) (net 20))
 (segment (start -30.766396 -44.127819) (end -29.310577 -42.672) (width 0.5588) (layer F.Cu) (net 21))
 (segment (start -21.850222 -41.654551) (end -22.485221 -42.28955) (width 0.5588) (layer F.Cu) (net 21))
 (segment (start -22.485221 -42.28955) (end -28.928127 -42.28955) (width 0.5588) (layer F.Cu) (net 21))
 (segment (start -28.928127 -42.28955) (end -29.310577 -42.672) (width 0.5588) (layer F.Cu) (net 21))
 (segment (start -21.850222 -41.654551) (end -21.850222 -38.455597) (width 0.5588) (layer F.Cu) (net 21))
 (segment (start -21.850222 -38.455597) (end -20.950074 -37.555449) (width 0.5588) (layer F.Cu) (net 21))
 (segment (start -53.6 4.58) (end -50.3 4.58) (width 0.5588) (layer F.Cu) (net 22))
 (segment (start -50.3 4.58) (end -48.346201 2.626201) (width 0.5588) (layer F.Cu) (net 22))
 (segment (start -47 -1.905) (end -48.346201 -0.558799) (width 0.5588) (layer F.Cu) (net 22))
 (segment (start -48.346201 -0.558799) (end -48.346201 2.626201) (width 0.5588) (layer F.Cu) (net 22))
 (segment (start -53.485 4.58) (end -53.6 4.58) (width 0.5588) (layer F.Cu) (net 22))
 (segment (start -43 -0.635) (end -45.73 -0.635) (width 0.5588) (layer F.Cu) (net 22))
 (segment (start -45.73 -0.635) (end -47 -1.905) (width 0.5588) (layer F.Cu) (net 22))
 (segment (start -25.149778 39.749551) (end -25.149778 40.812225) (width 0.4488) (layer F.Cu) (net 23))
 (segment (start -25.149778 40.812225) (end -22.833604 43.128399) (width 0.4488) (layer F.Cu) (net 23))
 (segment (start -22.833604 43.128399) (end -22.833604 47.970429) (width 0.4488) (layer F.Cu) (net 23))
 (segment (start -22.833604 47.970429) (end -22.833604 48.705514) (width 0.4488) (layer F.Cu) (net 23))
 (segment (start -22.049926 36.920449) (end -24.879028 39.749551) (width 0.4488) (layer F.Cu) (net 23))
 (segment (start -24.879028 39.749551) (end -25.149778 39.749551) (width 0.4488) (layer F.Cu) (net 23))
 (segment (start 21.861156 57.06349) (end 22.120964 56.91349) (width 0.25) (layer F.Cu) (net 4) (status 30)))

